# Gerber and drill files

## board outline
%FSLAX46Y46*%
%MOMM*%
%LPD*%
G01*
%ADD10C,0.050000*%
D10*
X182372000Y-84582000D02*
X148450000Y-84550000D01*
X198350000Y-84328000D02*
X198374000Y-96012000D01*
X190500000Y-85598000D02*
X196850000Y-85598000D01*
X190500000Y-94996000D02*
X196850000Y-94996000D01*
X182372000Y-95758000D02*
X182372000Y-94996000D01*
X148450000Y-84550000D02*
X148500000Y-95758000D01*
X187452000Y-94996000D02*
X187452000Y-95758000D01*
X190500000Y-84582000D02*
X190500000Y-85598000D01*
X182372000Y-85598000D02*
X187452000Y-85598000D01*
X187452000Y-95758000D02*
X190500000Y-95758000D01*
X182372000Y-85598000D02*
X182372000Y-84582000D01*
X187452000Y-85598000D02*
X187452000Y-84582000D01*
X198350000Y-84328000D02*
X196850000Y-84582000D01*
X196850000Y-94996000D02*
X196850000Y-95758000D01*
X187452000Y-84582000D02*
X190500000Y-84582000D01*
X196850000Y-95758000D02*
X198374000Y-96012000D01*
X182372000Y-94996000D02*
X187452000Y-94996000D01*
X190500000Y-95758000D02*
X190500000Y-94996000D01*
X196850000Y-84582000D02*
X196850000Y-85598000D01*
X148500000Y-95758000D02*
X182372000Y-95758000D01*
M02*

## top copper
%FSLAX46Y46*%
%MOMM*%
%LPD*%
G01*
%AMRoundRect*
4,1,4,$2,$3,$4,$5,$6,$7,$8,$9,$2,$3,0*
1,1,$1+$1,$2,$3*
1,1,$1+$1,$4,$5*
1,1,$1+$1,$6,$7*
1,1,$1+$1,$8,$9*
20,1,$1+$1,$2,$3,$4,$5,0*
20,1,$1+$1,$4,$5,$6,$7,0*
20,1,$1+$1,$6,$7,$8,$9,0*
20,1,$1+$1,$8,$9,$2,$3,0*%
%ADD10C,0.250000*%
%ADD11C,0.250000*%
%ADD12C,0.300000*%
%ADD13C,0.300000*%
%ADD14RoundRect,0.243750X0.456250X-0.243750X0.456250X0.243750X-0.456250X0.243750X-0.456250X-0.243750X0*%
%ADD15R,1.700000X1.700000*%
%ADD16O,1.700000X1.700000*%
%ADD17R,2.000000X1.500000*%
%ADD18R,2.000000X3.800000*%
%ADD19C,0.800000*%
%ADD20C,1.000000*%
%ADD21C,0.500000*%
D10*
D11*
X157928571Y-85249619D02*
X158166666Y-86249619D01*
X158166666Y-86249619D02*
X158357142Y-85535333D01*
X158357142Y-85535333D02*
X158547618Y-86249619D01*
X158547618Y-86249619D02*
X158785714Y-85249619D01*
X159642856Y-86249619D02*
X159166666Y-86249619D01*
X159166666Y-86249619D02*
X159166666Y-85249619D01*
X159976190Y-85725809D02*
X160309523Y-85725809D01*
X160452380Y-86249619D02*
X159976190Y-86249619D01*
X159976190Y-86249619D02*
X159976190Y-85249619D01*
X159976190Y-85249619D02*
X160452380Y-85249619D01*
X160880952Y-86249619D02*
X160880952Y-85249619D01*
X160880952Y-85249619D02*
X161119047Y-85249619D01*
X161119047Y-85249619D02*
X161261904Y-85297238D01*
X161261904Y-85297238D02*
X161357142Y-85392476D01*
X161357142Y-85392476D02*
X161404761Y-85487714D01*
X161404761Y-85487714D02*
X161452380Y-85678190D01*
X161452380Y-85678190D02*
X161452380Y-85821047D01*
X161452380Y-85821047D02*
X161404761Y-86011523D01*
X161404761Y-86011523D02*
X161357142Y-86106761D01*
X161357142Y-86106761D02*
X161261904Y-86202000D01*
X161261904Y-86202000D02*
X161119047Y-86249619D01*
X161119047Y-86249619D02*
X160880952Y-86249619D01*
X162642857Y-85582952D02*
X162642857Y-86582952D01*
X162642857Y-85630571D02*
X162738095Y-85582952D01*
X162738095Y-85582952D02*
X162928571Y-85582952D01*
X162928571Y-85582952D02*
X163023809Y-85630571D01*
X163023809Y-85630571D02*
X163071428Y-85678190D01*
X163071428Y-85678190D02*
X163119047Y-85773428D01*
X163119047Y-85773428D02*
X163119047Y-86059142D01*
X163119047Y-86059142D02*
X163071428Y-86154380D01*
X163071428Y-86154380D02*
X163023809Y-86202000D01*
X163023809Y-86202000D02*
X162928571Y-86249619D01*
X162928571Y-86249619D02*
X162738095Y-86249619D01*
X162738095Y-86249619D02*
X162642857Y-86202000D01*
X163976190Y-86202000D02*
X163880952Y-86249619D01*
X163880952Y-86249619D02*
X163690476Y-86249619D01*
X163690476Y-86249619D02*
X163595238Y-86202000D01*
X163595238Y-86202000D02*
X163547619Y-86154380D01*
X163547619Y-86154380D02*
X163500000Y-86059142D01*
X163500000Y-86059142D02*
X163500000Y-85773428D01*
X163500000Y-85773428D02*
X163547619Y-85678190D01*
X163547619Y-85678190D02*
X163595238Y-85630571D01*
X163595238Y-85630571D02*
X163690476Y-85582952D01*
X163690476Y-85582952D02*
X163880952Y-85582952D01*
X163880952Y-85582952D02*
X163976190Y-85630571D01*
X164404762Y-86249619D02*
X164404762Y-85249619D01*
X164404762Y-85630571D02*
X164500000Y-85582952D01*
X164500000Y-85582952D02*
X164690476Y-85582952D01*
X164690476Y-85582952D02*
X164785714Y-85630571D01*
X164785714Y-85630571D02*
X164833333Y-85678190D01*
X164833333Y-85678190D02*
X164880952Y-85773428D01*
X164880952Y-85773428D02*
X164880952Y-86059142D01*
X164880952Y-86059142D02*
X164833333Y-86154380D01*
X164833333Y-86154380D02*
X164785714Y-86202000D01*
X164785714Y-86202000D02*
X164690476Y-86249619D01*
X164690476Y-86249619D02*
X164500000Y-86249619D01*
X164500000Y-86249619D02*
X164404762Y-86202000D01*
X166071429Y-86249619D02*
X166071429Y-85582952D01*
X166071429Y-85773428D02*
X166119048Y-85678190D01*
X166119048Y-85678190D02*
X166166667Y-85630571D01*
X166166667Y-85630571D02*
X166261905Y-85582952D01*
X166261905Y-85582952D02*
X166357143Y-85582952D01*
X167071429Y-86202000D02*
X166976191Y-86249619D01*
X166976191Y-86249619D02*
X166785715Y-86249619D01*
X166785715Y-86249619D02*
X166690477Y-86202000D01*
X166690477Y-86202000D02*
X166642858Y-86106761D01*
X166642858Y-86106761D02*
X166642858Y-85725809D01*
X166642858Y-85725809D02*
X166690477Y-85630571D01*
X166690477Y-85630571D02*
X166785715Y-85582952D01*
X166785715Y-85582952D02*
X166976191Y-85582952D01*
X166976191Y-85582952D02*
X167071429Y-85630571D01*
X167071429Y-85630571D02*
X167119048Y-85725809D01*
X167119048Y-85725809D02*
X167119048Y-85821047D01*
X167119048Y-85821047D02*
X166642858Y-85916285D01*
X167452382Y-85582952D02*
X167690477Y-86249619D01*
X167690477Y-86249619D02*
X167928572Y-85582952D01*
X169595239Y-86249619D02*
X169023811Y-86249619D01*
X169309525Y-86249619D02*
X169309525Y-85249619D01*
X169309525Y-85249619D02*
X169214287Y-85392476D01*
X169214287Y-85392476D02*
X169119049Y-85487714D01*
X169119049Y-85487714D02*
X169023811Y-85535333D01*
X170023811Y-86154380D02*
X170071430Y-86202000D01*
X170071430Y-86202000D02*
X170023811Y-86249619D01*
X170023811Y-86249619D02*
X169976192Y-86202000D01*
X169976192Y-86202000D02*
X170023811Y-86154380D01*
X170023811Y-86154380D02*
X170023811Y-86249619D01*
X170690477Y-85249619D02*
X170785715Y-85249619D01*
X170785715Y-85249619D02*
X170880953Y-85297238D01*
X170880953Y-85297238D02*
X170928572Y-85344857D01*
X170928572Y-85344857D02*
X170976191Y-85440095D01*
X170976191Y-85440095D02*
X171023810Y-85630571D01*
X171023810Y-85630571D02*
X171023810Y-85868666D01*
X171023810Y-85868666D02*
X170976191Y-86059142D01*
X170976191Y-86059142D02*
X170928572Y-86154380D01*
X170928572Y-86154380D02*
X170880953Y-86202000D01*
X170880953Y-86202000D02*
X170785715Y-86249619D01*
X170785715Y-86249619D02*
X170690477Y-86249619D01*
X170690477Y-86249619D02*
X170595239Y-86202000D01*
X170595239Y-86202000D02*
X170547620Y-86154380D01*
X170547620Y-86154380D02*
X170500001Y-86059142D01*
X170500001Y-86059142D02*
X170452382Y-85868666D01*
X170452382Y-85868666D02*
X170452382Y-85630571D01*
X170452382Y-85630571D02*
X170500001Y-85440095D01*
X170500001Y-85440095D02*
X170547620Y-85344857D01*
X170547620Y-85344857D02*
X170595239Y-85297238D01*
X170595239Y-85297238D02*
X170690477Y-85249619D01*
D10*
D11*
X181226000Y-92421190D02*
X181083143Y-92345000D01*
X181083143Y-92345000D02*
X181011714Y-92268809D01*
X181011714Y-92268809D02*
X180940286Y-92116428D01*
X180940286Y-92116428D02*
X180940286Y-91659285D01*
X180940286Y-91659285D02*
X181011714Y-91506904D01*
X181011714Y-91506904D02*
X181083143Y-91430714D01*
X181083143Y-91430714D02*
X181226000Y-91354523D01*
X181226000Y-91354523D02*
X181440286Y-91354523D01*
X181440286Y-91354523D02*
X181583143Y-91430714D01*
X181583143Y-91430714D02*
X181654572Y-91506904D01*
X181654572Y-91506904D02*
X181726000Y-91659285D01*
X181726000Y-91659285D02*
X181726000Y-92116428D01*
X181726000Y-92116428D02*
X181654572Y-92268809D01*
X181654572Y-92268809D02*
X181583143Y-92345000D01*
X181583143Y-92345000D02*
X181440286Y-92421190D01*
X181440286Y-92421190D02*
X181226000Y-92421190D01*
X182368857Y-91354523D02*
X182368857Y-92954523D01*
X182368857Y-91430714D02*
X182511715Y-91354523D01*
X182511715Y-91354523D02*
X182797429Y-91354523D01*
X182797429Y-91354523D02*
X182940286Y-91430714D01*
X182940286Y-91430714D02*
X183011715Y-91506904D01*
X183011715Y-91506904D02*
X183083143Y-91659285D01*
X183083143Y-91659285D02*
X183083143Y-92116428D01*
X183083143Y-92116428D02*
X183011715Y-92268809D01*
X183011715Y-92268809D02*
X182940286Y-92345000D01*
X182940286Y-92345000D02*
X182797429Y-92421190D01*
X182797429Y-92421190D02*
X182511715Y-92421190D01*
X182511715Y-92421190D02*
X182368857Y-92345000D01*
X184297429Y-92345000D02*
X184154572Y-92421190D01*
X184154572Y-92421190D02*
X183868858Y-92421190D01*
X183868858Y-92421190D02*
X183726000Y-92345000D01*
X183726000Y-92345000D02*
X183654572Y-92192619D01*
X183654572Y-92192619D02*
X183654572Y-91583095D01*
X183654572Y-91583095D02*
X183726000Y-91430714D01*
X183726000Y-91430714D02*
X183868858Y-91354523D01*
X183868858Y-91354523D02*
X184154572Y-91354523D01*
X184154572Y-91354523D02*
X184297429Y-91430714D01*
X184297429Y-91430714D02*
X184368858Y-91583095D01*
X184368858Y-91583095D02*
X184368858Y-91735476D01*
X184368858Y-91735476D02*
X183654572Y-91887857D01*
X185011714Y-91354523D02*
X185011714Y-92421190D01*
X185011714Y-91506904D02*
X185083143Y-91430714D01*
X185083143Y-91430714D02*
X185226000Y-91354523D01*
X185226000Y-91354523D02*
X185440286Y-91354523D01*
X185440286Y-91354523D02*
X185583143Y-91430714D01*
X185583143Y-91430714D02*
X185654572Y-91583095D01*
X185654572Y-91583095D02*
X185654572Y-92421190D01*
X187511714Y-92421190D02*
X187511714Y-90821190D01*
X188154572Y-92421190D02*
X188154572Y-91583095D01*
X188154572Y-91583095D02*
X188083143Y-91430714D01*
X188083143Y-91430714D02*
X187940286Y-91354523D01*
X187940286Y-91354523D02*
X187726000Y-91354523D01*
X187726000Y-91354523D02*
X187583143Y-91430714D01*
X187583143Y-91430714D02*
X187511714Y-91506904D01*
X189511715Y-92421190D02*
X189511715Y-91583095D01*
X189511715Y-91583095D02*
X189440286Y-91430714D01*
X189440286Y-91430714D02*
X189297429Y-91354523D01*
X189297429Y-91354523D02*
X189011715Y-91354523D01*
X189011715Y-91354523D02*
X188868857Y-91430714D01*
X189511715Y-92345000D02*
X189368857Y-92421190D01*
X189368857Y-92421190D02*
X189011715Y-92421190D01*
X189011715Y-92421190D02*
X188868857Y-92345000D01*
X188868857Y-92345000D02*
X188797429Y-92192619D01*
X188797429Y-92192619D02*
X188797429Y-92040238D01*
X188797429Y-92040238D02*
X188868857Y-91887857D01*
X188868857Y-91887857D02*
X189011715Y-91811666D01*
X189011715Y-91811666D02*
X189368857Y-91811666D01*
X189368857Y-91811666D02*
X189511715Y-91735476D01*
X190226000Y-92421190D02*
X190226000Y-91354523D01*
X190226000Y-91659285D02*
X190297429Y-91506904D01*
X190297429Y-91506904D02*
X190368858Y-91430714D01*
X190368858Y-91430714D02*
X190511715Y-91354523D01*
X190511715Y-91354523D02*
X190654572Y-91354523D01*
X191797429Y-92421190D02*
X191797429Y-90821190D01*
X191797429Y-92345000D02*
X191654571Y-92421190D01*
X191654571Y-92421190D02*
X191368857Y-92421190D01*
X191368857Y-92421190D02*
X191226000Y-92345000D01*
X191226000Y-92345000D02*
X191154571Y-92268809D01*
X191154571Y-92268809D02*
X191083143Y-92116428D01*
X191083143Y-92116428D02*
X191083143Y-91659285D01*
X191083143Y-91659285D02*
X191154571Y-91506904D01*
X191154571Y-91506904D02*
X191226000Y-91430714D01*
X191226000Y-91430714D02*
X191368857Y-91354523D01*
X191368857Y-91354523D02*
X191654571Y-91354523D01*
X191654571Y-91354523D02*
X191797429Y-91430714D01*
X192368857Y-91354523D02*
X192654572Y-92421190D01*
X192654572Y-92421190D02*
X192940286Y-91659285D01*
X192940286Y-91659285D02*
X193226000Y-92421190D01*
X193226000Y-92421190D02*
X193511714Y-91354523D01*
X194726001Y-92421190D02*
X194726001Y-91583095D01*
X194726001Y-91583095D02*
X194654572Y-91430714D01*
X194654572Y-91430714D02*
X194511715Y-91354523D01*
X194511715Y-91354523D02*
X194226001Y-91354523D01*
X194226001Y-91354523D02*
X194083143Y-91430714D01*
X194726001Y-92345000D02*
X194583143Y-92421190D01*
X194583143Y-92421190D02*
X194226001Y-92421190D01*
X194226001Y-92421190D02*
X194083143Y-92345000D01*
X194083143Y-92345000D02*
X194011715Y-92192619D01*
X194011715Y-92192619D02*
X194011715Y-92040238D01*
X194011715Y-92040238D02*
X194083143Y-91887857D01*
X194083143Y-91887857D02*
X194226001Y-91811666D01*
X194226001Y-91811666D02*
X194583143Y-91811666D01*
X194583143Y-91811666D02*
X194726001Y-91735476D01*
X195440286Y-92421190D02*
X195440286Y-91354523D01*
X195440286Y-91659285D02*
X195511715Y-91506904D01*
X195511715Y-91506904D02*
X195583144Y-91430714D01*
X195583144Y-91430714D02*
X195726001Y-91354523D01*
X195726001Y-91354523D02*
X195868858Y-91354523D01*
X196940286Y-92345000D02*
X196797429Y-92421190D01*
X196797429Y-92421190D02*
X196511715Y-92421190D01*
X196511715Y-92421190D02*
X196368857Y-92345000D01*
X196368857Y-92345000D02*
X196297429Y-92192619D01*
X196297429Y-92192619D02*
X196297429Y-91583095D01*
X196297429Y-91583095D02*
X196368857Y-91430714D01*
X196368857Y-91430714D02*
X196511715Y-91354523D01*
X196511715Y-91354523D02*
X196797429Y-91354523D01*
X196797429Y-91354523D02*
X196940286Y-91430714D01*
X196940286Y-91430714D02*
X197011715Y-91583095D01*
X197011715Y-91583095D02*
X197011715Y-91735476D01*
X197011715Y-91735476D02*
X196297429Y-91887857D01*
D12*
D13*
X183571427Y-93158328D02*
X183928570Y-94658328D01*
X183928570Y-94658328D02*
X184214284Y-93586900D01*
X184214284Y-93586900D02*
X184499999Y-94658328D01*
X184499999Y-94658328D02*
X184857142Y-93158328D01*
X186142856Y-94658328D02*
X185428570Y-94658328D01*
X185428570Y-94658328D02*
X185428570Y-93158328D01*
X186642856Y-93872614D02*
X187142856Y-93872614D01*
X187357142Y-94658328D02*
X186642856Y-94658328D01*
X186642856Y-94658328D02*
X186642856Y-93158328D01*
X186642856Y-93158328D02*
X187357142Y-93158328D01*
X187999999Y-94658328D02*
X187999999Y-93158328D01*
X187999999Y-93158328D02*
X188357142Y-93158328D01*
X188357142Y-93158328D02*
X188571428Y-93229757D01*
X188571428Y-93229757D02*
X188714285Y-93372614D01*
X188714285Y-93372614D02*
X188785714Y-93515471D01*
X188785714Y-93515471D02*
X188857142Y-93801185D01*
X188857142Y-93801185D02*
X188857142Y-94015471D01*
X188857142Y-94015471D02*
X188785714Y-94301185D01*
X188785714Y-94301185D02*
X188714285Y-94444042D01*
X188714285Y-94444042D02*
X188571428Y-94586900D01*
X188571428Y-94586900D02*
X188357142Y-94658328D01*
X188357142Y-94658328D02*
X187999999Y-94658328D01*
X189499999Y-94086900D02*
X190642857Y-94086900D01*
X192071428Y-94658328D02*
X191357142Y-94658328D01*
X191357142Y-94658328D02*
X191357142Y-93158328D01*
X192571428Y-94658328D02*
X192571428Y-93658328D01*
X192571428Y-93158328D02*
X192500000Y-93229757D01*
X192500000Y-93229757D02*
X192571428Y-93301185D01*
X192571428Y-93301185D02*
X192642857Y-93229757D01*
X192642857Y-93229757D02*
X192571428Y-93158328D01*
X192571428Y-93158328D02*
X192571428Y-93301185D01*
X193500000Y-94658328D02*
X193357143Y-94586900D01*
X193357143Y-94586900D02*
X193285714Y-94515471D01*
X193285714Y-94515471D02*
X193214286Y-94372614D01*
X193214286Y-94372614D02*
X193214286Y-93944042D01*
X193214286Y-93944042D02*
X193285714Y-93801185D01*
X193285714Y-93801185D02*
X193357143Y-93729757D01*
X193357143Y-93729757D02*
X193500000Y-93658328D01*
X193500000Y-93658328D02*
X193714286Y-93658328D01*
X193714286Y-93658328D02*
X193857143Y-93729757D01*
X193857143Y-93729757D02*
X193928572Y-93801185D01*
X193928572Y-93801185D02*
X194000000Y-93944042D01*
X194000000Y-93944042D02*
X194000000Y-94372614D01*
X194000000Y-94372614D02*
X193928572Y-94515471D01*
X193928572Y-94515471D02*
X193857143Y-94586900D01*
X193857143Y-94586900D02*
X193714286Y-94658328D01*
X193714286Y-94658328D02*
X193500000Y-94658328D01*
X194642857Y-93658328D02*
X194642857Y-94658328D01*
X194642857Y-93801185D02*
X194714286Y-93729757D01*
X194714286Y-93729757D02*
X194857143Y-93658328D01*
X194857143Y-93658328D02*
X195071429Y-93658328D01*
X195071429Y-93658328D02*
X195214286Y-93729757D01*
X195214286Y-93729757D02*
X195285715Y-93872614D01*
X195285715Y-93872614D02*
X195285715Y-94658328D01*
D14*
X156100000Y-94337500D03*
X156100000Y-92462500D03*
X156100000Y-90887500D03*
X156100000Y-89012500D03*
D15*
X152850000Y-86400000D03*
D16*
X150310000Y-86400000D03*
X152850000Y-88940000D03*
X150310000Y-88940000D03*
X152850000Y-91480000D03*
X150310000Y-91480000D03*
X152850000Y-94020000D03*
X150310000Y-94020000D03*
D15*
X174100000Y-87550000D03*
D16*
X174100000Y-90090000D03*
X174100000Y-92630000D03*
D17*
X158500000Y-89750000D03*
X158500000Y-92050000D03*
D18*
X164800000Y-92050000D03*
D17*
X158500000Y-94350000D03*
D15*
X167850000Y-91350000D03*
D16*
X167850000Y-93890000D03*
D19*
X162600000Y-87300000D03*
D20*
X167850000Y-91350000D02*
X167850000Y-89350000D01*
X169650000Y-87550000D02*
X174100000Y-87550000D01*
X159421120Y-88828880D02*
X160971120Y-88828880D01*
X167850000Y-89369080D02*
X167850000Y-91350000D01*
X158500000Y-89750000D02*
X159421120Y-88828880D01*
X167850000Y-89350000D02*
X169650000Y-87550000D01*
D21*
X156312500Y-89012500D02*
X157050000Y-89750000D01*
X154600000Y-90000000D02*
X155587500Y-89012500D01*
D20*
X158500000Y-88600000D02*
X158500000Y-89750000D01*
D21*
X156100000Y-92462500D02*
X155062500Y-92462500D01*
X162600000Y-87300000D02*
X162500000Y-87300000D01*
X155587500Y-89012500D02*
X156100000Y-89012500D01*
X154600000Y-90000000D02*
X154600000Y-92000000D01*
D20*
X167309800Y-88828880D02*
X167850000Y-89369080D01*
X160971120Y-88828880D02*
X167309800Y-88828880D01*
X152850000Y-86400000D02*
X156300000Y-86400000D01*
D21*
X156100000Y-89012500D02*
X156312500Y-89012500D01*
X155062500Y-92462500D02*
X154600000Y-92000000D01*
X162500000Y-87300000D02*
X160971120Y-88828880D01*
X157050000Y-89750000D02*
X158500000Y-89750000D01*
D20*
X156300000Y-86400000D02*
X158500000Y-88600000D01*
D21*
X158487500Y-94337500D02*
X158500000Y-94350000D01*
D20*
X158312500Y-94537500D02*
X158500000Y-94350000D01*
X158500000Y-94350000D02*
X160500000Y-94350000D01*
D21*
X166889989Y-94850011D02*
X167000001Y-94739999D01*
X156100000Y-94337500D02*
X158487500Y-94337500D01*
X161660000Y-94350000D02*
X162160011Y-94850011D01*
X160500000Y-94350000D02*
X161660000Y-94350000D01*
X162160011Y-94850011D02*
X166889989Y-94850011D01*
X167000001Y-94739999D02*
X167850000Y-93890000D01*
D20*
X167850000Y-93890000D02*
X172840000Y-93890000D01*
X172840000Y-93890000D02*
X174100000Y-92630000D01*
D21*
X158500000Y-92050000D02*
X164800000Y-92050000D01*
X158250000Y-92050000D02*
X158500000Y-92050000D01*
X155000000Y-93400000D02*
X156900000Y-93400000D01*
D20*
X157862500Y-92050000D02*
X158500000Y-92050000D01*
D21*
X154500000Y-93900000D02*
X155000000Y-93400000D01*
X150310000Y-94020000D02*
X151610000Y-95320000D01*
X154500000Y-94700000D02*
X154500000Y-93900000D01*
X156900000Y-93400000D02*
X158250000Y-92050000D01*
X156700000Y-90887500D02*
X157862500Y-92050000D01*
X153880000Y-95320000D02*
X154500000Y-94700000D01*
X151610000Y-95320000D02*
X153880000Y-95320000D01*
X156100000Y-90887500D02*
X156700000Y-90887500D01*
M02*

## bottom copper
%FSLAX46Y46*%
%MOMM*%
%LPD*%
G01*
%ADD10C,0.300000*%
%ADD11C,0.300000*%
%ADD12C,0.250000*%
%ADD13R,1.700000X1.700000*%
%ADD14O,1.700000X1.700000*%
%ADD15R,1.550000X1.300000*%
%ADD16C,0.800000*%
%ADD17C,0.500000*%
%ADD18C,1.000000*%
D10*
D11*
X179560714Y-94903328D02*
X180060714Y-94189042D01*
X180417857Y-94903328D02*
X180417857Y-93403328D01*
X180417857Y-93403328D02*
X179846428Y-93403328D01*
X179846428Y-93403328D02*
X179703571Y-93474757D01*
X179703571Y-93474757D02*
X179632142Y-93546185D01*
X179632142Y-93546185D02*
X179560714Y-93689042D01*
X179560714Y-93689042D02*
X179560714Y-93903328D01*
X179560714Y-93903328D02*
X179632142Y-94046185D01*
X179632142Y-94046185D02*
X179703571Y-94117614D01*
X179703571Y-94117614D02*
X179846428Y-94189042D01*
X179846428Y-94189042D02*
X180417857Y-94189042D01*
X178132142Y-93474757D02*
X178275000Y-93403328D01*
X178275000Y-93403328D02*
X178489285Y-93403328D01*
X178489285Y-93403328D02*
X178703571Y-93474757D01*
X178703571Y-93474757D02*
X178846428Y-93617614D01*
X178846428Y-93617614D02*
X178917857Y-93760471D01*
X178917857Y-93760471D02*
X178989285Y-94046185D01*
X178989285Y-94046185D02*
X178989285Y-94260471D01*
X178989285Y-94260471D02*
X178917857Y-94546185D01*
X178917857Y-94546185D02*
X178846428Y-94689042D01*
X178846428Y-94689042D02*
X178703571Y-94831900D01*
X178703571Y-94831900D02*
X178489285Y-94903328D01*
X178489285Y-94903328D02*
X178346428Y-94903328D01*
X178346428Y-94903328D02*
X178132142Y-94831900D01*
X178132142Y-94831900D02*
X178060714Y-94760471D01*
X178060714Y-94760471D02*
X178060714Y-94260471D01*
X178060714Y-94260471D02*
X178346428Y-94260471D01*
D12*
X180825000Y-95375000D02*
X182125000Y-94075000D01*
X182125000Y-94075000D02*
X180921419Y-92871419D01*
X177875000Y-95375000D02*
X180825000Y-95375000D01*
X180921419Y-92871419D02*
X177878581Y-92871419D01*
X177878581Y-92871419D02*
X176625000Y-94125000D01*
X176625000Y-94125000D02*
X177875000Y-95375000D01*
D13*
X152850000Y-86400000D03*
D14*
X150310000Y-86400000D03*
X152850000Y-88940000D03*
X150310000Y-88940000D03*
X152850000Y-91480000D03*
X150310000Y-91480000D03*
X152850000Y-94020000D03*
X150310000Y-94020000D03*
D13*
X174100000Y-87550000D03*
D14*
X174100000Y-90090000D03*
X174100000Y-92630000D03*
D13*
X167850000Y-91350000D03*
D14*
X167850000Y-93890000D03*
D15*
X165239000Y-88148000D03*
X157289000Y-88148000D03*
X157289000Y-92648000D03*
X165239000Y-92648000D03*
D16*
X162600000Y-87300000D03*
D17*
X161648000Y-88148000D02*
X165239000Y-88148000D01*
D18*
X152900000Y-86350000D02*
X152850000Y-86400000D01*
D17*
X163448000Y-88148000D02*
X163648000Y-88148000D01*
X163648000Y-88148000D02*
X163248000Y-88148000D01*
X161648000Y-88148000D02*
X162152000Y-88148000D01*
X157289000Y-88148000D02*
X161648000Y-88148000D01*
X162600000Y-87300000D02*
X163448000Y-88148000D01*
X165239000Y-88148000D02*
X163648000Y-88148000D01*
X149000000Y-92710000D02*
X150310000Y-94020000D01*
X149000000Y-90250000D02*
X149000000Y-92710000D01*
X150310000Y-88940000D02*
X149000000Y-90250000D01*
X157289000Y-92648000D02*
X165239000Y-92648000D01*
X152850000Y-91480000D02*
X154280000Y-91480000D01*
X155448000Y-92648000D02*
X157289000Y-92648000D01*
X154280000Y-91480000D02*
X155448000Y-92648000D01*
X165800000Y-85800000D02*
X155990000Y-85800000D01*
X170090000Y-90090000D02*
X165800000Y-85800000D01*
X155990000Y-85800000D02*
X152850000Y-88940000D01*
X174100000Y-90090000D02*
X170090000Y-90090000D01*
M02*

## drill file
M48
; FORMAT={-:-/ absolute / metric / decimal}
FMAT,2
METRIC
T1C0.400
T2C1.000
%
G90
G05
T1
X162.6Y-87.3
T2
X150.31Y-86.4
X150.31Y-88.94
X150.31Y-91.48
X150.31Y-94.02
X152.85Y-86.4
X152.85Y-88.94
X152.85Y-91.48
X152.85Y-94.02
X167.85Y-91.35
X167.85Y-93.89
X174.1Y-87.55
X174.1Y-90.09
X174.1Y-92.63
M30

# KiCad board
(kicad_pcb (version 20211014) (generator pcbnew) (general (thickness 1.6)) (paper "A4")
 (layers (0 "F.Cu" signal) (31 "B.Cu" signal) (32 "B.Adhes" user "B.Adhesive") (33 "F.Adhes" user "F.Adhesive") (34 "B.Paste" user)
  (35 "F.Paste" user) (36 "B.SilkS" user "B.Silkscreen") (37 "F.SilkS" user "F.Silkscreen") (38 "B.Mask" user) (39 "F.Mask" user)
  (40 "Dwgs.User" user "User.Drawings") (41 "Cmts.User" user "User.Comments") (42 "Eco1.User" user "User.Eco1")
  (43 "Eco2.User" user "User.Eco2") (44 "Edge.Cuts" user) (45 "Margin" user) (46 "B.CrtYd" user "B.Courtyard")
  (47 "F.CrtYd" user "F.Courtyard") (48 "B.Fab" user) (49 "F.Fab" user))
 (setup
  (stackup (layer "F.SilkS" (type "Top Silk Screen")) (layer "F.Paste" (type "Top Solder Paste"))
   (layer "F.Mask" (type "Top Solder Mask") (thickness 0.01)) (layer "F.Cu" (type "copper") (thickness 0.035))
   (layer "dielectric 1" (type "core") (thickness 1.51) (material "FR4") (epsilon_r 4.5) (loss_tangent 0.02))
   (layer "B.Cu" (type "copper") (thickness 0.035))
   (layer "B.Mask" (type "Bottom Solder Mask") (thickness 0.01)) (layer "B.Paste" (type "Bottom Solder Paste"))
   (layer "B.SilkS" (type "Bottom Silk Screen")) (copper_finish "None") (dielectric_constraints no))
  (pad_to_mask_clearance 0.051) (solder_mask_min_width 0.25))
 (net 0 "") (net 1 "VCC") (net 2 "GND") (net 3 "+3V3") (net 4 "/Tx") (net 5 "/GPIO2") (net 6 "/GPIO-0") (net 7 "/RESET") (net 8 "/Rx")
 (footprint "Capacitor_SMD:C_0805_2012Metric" (layer "F.Cu") (at 156.1 93.4 90)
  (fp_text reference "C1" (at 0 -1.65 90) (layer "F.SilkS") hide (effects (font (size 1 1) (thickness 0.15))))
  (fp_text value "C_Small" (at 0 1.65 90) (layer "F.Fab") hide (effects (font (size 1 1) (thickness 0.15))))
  (pad "1" smd roundrect locked (at -0.9375 0 90) (size 0.975 1.4) (layers "F.Cu" "F.Paste" "F.Mask") (roundrect_rratio 0.25) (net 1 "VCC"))
  (pad "2" smd roundrect locked (at 0.9375 0 90) (size 0.975 1.4) (layers "F.Cu" "F.Paste" "F.Mask") (roundrect_rratio 0.25) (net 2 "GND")))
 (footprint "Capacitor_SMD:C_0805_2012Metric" (layer "F.Cu") (at 156.1 89.95 90)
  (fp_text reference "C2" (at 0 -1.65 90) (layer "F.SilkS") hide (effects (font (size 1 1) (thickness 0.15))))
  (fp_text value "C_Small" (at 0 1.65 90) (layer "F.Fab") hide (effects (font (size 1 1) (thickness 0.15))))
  (pad "1" smd roundrect locked (at -0.9375 0 90) (size 0.975 1.4) (layers "F.Cu" "F.Paste" "F.Mask") (roundrect_rratio 0.25) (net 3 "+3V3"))
  (pad "2" smd roundrect locked (at 0.9375 0 90) (size 0.975 1.4) (layers "F.Cu" "F.Paste" "F.Mask") (roundrect_rratio 0.25) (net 2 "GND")))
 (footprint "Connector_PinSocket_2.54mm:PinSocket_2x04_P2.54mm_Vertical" (layer "F.Cu") (at 152.85 86.4)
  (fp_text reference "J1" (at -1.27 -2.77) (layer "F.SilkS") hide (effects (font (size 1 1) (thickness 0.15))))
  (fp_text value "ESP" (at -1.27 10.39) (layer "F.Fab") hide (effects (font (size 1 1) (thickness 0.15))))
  (pad "1" thru_hole rect locked (at 0 0) (size 1.7 1.7) (drill 1) (layers *.Cu *.Mask) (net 2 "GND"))
  (pad "2" thru_hole oval locked (at -2.54 0) (size 1.7 1.7) (drill 1) (layers *.Cu *.Mask) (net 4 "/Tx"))
  (pad "3" thru_hole oval locked (at 0 2.54) (size 1.7 1.7) (drill 1) (layers *.Cu *.Mask) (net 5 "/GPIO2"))
  (pad "4" thru_hole oval locked (at -2.54 2.54) (size 1.7 1.7) (drill 1) (layers *.Cu *.Mask) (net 3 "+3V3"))
  (pad "5" thru_hole oval locked (at 0 5.08) (size 1.7 1.7) (drill 1) (layers *.Cu *.Mask) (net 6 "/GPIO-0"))
  (pad "6" thru_hole oval locked (at -2.54 5.08) (size 1.7 1.7) (drill 1) (layers *.Cu *.Mask) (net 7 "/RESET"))
  (pad "7" thru_hole oval locked (at 0 7.62) (size 1.7 1.7) (drill 1) (layers *.Cu *.Mask) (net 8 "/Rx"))
  (pad "8" thru_hole oval locked (at -2.54 7.62) (size 1.7 1.7) (drill 1) (layers *.Cu *.Mask) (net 3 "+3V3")))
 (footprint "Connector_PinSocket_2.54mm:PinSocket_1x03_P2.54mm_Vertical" (layer "F.Cu") (at 174.1 87.55)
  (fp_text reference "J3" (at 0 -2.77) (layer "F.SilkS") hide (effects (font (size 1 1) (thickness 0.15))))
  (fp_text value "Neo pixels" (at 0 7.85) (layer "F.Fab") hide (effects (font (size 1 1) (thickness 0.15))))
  (pad "1" thru_hole rect locked (at 0 0) (size 1.7 1.7) (drill 1) (layers *.Cu *.Mask) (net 2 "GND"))
  (pad "2" thru_hole oval locked (at 0 2.54) (size 1.7 1.7) (drill 1) (layers *.Cu *.Mask) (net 5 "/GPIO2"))
  (pad "3" thru_hole oval locked (at 0 5.08) (size 1.7 1.7) (drill 1) (layers *.Cu *.Mask) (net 1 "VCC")))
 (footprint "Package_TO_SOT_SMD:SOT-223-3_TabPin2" (layer "F.Cu") (at 161.65 92.05)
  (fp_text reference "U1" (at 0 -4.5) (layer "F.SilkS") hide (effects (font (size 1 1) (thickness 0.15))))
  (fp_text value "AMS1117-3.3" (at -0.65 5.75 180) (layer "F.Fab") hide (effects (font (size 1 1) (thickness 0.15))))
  (pad "1" smd rect locked (at -3.15 -2.3) (size 2 1.5) (layers "F.Cu" "F.Paste" "F.Mask") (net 2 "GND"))
  (pad "2" smd rect locked (at -3.15 0) (size 2 1.5) (layers "F.Cu" "F.Paste" "F.Mask") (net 3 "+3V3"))
  (pad "2" smd rect locked (at 3.15 0) (size 2 3.8) (layers "F.Cu" "F.Paste" "F.Mask") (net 3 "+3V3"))
  (pad "3" smd rect locked (at -3.15 2.3) (size 2 1.5) (layers "F.Cu" "F.Paste" "F.Mask") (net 1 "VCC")))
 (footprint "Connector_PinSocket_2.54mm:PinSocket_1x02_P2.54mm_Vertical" (layer "F.Cu") (at 167.85 91.35)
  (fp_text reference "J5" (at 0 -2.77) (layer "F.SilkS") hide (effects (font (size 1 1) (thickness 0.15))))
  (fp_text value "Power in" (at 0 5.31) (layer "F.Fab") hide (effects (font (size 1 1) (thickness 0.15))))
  (pad "1" thru_hole rect locked (at 0 0) (size 1.7 1.7) (drill 1) (layers *.Cu *.Mask) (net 2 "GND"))
  (pad "2" thru_hole oval locked (at 0 2.54) (size 1.7 1.7) (drill 1) (layers *.Cu *.Mask) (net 1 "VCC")))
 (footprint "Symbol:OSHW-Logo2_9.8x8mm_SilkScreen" (layer "F.Cu") (at 189 88.821846)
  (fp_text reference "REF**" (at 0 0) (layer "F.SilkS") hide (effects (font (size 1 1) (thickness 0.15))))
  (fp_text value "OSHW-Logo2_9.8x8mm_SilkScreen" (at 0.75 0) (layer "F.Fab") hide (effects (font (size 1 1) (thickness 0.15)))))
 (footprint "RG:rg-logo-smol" (layer "F.Cu") (at 179.3 94.1 180)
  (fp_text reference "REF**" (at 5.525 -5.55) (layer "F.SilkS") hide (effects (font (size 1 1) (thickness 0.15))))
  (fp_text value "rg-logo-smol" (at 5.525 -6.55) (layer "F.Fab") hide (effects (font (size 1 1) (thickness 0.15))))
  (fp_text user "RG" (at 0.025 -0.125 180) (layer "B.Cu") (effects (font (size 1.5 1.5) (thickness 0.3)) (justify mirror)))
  (fp_line (start -1.525 -1.275) (end -2.825 0.025) (layer "B.Cu") (width 0.25))
  (fp_line (start -2.825 0.025) (end -1.621419 1.228581) (layer "B.Cu") (width 0.25))
  (fp_line (start 1.425 -1.275) (end -1.525 -1.275) (layer "B.Cu") (width 0.25))
  (fp_line (start -1.621419 1.228581) (end 1.421419 1.228581) (layer "B.Cu") (width 0.25))
  (fp_line (start 1.421419 1.228581) (end 2.675 -0.025) (layer "B.Cu") (width 0.25))
  (fp_line (start 2.675 -0.025) (end 1.425 -1.275) (layer "B.Cu") (width 0.25)))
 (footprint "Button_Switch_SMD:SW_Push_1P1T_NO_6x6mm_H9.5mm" (layer "B.Cu") (at 161.264 90.398 180)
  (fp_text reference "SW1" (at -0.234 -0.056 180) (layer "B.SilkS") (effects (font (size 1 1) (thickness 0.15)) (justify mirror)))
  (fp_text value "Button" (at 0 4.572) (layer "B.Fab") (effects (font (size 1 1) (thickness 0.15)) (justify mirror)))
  (pad "1" smd rect locked (at -3.975 2.25 180) (size 1.55 1.3) (layers "B.Cu" "B.Paste" "B.Mask") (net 2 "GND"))
  (pad "1" smd rect locked (at 3.975 2.25 180) (size 1.55 1.3) (layers "B.Cu" "B.Paste" "B.Mask") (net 2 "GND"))
  (pad "2" smd rect locked (at 3.975 -2.25 180) (size 1.55 1.3) (layers "B.Cu" "B.Paste" "B.Mask") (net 6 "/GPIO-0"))
  (pad "2" smd rect locked (at -3.975 -2.25 180) (size 1.55 1.3) (layers "B.Cu" "B.Paste" "B.Mask") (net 6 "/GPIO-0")))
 (gr_line (start 182.372 84.582) (end 148.45 84.55) (layer "Edge.Cuts") (width 0.05))
 (gr_line (start 198.35 84.328) (end 198.374 96.012) (layer "Edge.Cuts") (width 0.05))
 (gr_line (start 190.5 85.598) (end 196.85 85.598) (layer "Edge.Cuts") (width 0.05))
 (gr_line (start 190.5 94.996) (end 196.85 94.996) (layer "Edge.Cuts") (width 0.05))
 (gr_line (start 182.372 95.758) (end 182.372 94.996) (layer "Edge.Cuts") (width 0.05))
 (gr_line (start 148.45 84.55) (end 148.5 95.758) (layer "Edge.Cuts") (width 0.05))
 (gr_line (start 187.452 94.996) (end 187.452 95.758) (layer "Edge.Cuts") (width 0.05))
 (gr_line (start 190.5 84.582) (end 190.5 85.598) (layer "Edge.Cuts") (width 0.05))
 (gr_line (start 182.372 85.598) (end 187.452 85.598) (layer "Edge.Cuts") (width 0.05))
 (gr_line (start 187.452 95.758) (end 190.5 95.758) (layer "Edge.Cuts") (width 0.05))
 (gr_line (start 182.372 85.598) (end 182.372 84.582) (layer "Edge.Cuts") (width 0.05))
 (gr_line (start 187.452 85.598) (end 187.452 84.582) (layer "Edge.Cuts") (width 0.05))
 (gr_line (start 198.35 84.328) (end 196.85 84.582) (layer "Edge.Cuts") (width 0.05))
 (gr_line (start 196.85 94.996) (end 196.85 95.758) (layer "Edge.Cuts") (width 0.05))
 (gr_line (start 187.452 84.582) (end 190.5 84.582) (layer "Edge.Cuts") (width 0.05))
 (gr_line (start 196.85 95.758) (end 198.374 96.012) (layer "Edge.Cuts") (width 0.05))
 (gr_line (start 182.372 94.996) (end 187.452 94.996) (layer "Edge.Cuts") (width 0.05))
 (gr_line (start 190.5 95.758) (end 190.5 94.996) (layer "Edge.Cuts") (width 0.05))
 (gr_line (start 196.85 84.582) (end 196.85 85.598) (layer "Edge.Cuts") (width 0.05))
 (gr_line (start 148.5 95.758) (end 182.372 95.758) (layer "Edge.Cuts") (width 0.05))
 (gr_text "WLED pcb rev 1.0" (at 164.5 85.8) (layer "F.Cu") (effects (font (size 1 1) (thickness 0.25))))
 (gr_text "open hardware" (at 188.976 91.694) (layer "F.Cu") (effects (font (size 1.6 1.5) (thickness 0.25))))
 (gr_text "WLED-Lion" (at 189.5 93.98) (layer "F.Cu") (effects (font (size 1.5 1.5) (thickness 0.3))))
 (segment (start 167.85 91.35) (end 167.85 89.35) (width 1) (layer "F.Cu") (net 2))
 (segment (start 169.65 87.55) (end 174.1 87.55) (width 1) (layer "F.Cu") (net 2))
 (segment (start 159.42112 88.82888) (end 160.97112 88.82888) (width 1) (layer "F.Cu") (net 2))
 (segment (start 167.85 89.36908) (end 167.85 91.35) (width 1) (layer "F.Cu") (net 2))
 (segment (start 158.5 89.75) (end 159.42112 88.82888) (width 1) (layer "F.Cu") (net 2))
 (segment (start 167.85 89.35) (end 169.65 87.55) (width 1) (layer "F.Cu") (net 2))
 (segment (start 156.3125 89.0125) (end 157.05 89.75) (width 0.5) (layer "F.Cu") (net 2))
 (segment (start 154.6 90) (end 155.5875 89.0125) (width 0.5) (layer "F.Cu") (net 2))
 (segment (start 158.5 88.6) (end 158.5 89.75) (width 1) (layer "F.Cu") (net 2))
 (segment (start 156.1 92.4625) (end 155.0625 92.4625) (width 0.5) (layer "F.Cu") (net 2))
 (segment (start 162.6 87.3) (end 162.5 87.3) (width 0.5) (layer "F.Cu") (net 2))
 (segment (start 155.5875 89.0125) (end 156.1 89.0125) (width 0.5) (layer "F.Cu") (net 2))
 (segment (start 154.6 90) (end 154.6 92) (width 0.5) (layer "F.Cu") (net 2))
 (segment (start 167.3098 88.82888) (end 167.85 89.36908) (width 1) (layer "F.Cu") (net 2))
 (segment (start 160.97112 88.82888) (end 167.3098 88.82888) (width 1) (layer "F.Cu") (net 2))
 (segment (start 152.85 86.4) (end 156.3 86.4) (width 1) (layer "F.Cu") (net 2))
 (segment (start 156.1 89.0125) (end 156.3125 89.0125) (width 0.5) (layer "F.Cu") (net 2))
 (segment (start 155.0625 92.4625) (end 154.6 92) (width 0.5) (layer "F.Cu") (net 2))
 (segment (start 162.5 87.3) (end 160.97112 88.82888) (width 0.5) (layer "F.Cu") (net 2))
 (segment (start 157.05 89.75) (end 158.5 89.75) (width 0.5) (layer "F.Cu") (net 2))
 (segment (start 156.3 86.4) (end 158.5 88.6) (width 1) (layer "F.Cu") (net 2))
 (via (at 162.6 87.3) (size 0.8) (drill 0.4) (layers "F.Cu" "B.Cu") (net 2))
 (segment (start 161.648 88.148) (end 165.239 88.148) (width 0.5) (layer "B.Cu") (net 2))
 (segment (start 152.9 86.35) (end 152.85 86.4) (width 1) (layer "B.Cu") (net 2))
 (segment (start 163.448 88.148) (end 163.648 88.148) (width 0.5) (layer "B.Cu") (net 2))
 (segment (start 163.648 88.148) (end 163.248 88.148) (width 0.5) (layer "B.Cu") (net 2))
 (segment (start 161.648 88.148) (end 162.152 88.148) (width 0.5) (layer "B.Cu") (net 2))
 (segment (start 157.289 88.148) (end 161.648 88.148) (width 0.5) (layer "B.Cu") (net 2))
 (segment (start 162.6 87.3) (end 163.448 88.148) (width 0.5) (layer "B.Cu") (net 2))
 (segment (start 165.239 88.148) (end 163.648 88.148) (width 0.5) (layer "B.Cu") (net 2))
 (segment (start 158.4875 94.3375) (end 158.5 94.35) (width 0.5) (layer "F.Cu") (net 1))
 (segment (start 158.3125 94.5375) (end 158.5 94.35) (width 1) (layer "F.Cu") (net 1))
 (segment (start 158.5 94.35) (end 160.5 94.35) (width 1) (layer "F.Cu") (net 1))
 (segment (start 166.889989 94.850011) (end 167.000001 94.739999) (width 0.5) (layer "F.Cu") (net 1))
 (segment (start 156.1 94.3375) (end 158.4875 94.3375) (width 0.5) (layer "F.Cu") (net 1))
 (segment (start 161.66 94.35) (end 162.160011 94.850011) (width 0.5) (layer "F.Cu") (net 1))
 (segment (start 160.5 94.35) (end 161.66 94.35) (width 0.5) (layer "F.Cu") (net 1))
 (segment (start 162.160011 94.850011) (end 166.889989 94.850011) (width 0.5) (layer "F.Cu") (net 1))
 (segment (start 167.000001 94.739999) (end 167.85 93.89) (width 0.5) (layer "F.Cu") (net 1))
 (segment (start 167.85 93.89) (end 172.84 93.89) (width 1) (layer "F.Cu") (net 1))
 (segment (start 172.84 93.89) (end 174.1 92.63) (width 1) (layer "F.Cu") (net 1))
 (segment (start 158.5 92.05) (end 164.8 92.05) (width 0.5) (layer "F.Cu") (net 3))
 (segment (start 158.25 92.05) (end 158.5 92.05) (width 0.5) (layer "F.Cu") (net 3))
 (segment (start 155 93.4) (end 156.9 93.4) (width 0.5) (layer "F.Cu") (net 3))
 (segment (start 157.8625 92.05) (end 158.5 92.05) (width 1) (layer "F.Cu") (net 3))
 (segment (start 154.5 93.9) (end 155 93.4) (width 0.5) (layer "F.Cu") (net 3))
 (segment (start 150.31 94.02) (end 151.61 95.32) (width 0.5) (layer "F.Cu") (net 3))
 (segment (start 154.5 94.7) (end 154.5 93.9) (width 0.5) (layer "F.Cu") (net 3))
 (segment (start 156.9 93.4) (end 158.25 92.05) (width 0.5) (layer "F.Cu") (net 3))
 (segment (start 156.7 90.8875) (end 157.8625 92.05) (width 0.5) (layer "F.Cu") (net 3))
 (segment (start 153.88 95.32) (end 154.5 94.7) (width 0.5) (layer "F.Cu") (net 3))
 (segment (start 151.61 95.32) (end 153.88 95.32) (width 0.5) (layer "F.Cu") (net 3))
 (segment (start 156.1 90.8875) (end 156.7 90.8875) (width 0.5) (layer "F.Cu") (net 3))
 (segment (start 149 92.71) (end 150.31 94.02) (width 0.5) (layer "B.Cu") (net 3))
 (segment (start 149 90.25) (end 149 92.71) (width 0.5) (layer "B.Cu") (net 3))
 (segment (start 150.31 88.94) (end 149 90.25) (width 0.5) (layer "B.Cu") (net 3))
 (segment (start 157.289 92.648) (end 165.239 92.648) (width 0.5) (layer "B.Cu") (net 6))
 (segment (start 152.85 91.48) (end 154.28 91.48) (width 0.5) (layer "B.Cu") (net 6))
 (segment (start 155.448 92.648) (end 157.289 92.648) (width 0.5) (layer "B.Cu") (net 6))
 (segment (start 154.28 91.48) (end 155.448 92.648) (width 0.5) (layer "B.Cu") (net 6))
 (segment (start 165.8 85.8) (end 155.99 85.8) (width 0.5) (layer "B.Cu") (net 5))
 (segment (start 170.09 90.09) (end 165.8 85.8) (width 0.5) (layer "B.Cu") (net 5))
 (segment (start 155.99 85.8) (end 152.85 88.94) (width 0.5) (layer "B.Cu") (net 5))
 (segment (start 174.1 90.09) (end 170.09 90.09) (width 0.5) (layer "B.Cu") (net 5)))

